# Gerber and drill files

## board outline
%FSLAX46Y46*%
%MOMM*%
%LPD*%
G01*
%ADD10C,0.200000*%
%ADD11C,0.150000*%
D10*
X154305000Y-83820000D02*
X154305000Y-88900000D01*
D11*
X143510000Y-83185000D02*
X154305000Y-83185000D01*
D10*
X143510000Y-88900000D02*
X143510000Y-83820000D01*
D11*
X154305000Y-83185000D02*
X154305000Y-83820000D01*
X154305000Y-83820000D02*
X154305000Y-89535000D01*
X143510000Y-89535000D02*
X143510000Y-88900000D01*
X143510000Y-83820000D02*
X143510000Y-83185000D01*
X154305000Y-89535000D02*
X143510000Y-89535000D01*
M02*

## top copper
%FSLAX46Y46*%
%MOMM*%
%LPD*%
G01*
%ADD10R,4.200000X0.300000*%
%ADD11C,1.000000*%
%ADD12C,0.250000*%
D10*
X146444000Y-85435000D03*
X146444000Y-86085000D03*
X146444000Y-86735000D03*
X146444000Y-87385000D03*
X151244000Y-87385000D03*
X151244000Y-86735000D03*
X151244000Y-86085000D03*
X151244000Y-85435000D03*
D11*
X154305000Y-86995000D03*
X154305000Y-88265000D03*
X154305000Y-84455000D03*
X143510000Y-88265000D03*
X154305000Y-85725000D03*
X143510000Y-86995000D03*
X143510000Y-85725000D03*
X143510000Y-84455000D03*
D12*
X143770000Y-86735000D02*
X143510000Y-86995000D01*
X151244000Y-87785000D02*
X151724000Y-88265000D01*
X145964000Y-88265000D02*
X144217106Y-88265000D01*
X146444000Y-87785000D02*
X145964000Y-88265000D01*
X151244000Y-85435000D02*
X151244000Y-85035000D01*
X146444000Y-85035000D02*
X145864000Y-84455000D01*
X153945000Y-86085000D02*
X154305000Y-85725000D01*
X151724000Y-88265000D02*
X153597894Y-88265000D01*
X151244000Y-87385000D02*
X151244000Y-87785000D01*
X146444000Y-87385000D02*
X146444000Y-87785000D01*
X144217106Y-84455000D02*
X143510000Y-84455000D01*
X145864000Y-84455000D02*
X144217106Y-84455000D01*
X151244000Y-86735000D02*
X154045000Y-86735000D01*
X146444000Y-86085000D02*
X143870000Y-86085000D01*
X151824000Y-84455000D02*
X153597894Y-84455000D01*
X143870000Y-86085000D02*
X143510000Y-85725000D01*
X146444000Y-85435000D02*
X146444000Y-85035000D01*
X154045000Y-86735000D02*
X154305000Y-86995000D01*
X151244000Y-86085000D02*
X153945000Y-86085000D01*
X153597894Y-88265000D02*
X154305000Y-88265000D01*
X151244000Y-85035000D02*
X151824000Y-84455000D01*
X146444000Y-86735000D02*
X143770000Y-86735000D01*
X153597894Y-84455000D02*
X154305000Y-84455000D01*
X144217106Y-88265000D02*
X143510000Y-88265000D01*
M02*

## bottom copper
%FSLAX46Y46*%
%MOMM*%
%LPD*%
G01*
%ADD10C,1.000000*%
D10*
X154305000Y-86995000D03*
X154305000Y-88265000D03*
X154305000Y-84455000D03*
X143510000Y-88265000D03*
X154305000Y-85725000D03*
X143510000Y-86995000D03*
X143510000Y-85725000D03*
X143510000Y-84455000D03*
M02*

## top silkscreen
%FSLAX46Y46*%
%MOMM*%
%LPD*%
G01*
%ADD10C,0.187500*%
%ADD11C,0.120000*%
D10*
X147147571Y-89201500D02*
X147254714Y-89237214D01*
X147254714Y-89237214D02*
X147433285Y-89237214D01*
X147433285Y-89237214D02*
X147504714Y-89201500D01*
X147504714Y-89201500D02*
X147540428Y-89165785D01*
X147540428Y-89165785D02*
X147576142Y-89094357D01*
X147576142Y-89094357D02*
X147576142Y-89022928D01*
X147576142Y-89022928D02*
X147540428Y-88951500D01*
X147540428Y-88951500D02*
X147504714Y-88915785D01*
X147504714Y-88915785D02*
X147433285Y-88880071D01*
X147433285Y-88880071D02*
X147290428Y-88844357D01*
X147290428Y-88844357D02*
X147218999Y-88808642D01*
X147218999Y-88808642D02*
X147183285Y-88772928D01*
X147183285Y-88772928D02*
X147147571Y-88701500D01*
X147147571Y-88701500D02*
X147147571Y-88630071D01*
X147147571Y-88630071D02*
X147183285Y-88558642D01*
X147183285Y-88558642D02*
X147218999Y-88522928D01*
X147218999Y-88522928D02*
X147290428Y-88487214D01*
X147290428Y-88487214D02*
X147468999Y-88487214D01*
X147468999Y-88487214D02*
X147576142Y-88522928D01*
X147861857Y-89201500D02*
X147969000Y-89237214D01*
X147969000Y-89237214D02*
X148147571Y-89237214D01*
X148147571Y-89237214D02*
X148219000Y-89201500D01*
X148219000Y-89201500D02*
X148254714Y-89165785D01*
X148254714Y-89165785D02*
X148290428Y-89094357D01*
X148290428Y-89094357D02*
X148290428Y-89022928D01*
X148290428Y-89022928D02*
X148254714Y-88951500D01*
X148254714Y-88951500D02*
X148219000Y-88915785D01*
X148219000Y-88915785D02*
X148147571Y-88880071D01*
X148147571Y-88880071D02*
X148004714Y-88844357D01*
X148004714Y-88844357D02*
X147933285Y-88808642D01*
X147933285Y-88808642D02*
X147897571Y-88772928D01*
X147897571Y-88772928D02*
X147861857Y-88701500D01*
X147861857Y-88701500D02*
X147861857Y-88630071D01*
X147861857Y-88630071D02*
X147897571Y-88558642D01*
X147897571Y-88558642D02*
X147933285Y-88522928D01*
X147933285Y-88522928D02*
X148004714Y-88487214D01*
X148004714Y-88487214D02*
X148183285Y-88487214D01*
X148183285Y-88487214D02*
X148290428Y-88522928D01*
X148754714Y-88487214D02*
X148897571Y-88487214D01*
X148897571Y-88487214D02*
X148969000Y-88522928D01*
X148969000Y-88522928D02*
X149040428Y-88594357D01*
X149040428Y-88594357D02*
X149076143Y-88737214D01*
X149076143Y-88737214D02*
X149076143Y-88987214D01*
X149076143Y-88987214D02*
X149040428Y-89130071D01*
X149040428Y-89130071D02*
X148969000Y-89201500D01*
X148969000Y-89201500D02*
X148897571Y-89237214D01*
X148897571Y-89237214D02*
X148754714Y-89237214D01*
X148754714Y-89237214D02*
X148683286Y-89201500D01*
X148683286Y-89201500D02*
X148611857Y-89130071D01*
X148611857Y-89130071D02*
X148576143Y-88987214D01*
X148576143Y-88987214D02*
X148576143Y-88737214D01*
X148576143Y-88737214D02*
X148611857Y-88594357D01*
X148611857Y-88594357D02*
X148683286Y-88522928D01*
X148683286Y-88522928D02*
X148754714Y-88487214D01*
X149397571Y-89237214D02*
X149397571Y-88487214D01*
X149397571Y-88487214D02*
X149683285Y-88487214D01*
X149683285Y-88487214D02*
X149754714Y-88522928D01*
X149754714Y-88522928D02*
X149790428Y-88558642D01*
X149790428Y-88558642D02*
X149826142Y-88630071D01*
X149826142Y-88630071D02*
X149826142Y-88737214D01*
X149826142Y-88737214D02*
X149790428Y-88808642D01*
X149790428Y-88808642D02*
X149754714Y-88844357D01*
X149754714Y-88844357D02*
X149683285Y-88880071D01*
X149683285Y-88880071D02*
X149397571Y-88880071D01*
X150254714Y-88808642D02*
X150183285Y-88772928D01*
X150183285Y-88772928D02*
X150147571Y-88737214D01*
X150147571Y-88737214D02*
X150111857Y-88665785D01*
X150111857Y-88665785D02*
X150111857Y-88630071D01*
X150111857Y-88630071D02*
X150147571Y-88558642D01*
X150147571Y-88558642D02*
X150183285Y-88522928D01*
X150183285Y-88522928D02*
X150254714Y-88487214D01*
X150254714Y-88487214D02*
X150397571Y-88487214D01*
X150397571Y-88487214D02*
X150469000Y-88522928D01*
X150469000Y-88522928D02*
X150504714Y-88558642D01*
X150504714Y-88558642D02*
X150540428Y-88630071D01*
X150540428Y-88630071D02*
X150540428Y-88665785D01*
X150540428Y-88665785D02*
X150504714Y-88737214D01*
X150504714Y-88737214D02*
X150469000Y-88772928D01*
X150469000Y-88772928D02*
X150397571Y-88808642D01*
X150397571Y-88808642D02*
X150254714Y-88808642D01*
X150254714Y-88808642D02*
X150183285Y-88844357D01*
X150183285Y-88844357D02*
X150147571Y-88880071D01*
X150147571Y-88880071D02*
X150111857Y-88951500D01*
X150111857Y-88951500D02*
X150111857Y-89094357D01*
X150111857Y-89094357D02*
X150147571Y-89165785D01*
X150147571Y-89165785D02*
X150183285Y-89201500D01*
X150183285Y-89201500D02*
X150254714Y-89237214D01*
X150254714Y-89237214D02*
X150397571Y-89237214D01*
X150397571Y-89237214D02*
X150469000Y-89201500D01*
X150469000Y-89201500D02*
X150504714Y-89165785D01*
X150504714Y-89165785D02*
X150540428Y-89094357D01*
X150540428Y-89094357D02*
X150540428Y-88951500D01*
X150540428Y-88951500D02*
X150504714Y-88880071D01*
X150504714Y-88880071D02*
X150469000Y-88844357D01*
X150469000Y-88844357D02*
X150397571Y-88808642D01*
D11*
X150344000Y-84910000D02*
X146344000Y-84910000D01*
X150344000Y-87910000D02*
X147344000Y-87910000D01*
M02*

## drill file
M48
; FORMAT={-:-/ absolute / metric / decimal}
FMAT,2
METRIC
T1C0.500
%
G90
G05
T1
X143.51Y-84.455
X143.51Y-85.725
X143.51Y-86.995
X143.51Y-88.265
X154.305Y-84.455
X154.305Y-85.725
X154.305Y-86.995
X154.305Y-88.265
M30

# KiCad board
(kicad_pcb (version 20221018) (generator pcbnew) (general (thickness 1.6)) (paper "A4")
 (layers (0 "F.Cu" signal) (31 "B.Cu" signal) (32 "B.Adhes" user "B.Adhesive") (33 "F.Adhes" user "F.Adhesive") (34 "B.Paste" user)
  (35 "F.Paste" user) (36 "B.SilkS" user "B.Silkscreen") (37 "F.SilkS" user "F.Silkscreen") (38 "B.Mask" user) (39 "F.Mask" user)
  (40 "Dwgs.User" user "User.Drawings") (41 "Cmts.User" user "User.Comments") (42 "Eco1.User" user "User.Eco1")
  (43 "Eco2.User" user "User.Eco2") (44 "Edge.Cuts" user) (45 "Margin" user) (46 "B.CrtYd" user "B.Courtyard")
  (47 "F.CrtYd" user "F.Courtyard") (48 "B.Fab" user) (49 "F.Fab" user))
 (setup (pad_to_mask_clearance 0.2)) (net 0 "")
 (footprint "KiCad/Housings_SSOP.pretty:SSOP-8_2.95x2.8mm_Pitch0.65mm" (layer "F.Cu") (at 148.844 86.41)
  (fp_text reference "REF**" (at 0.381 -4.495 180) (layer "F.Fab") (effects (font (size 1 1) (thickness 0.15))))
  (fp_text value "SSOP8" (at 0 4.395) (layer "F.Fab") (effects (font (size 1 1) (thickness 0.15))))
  (fp_line (start 1.5 -1.5) (end -2.5 -1.5) (stroke (width 0.12) (type solid)) (layer "F.SilkS"))
  (fp_line (start 1.5 1.5) (end -1.5 1.5) (stroke (width 0.12) (type solid)) (layer "F.SilkS"))
  (pad "1" smd rect (at -2.4 -0.975 270) (size 0.3 4.2) (layers "F.Cu" "F.Paste" "F.Mask"))
  (pad "2" smd rect (at -2.4 -0.325 270) (size 0.3 4.2) (layers "F.Cu" "F.Paste" "F.Mask"))
  (pad "3" smd rect (at -2.4 0.325 270) (size 0.3 4.2) (layers "F.Cu" "F.Paste" "F.Mask"))
  (pad "4" smd rect (at -2.4 0.975 270) (size 0.3 4.2) (layers "F.Cu" "F.Paste" "F.Mask"))
  (pad "5" smd rect (at 2.4 0.975 270) (size 0.3 4.2) (layers "F.Cu" "F.Paste" "F.Mask"))
  (pad "6" smd rect (at 2.4 0.325 270) (size 0.3 4.2) (layers "F.Cu" "F.Paste" "F.Mask"))
  (pad "7" smd rect (at 2.4 -0.325 270) (size 0.3 4.2) (layers "F.Cu" "F.Paste" "F.Mask"))
  (pad "8" smd rect (at 2.4 -0.975 270) (size 0.3 4.2) (layers "F.Cu" "F.Paste" "F.Mask")))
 (gr_line (start 154.305 83.82) (end 154.305 88.9) (stroke (width 0.2) (type solid)) (layer "Edge.Cuts"))
 (gr_line (start 143.51 83.185) (end 154.305 83.185) (stroke (width 0.15) (type solid)) (layer "Edge.Cuts"))
 (gr_line (start 143.51 88.9) (end 143.51 83.82) (stroke (width 0.2) (type solid)) (layer "Edge.Cuts"))
 (gr_line (start 154.305 83.185) (end 154.305 83.82) (stroke (width 0.15) (type solid)) (layer "Edge.Cuts"))
 (gr_line (start 154.305 83.82) (end 154.305 89.535) (stroke (width 0.15) (type solid)) (layer "Edge.Cuts"))
 (gr_line (start 143.51 89.535) (end 143.51 88.9) (stroke (width 0.15) (type solid)) (layer "Edge.Cuts"))
 (gr_line (start 143.51 83.82) (end 143.51 83.185) (stroke (width 0.15) (type solid)) (layer "Edge.Cuts"))
 (gr_line (start 154.305 89.535) (end 143.51 89.535) (stroke (width 0.15) (type solid)) (layer "Edge.Cuts"))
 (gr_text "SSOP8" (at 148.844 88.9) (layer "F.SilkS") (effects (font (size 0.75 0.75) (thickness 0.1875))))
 (segment (start 143.77 86.735) (end 143.51 86.995) (width 0.25) (layer "F.Cu") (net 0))
 (segment (start 151.244 87.785) (end 151.724 88.265) (width 0.25) (layer "F.Cu") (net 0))
 (segment (start 145.964 88.265) (end 144.217106 88.265) (width 0.25) (layer "F.Cu") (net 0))
 (segment (start 146.444 87.785) (end 145.964 88.265) (width 0.25) (layer "F.Cu") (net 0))
 (segment (start 151.244 85.435) (end 151.244 85.035) (width 0.25) (layer "F.Cu") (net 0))
 (segment (start 146.444 85.035) (end 145.864 84.455) (width 0.25) (layer "F.Cu") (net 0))
 (segment (start 153.945 86.085) (end 154.305 85.725) (width 0.25) (layer "F.Cu") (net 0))
 (segment (start 151.724 88.265) (end 153.597894 88.265) (width 0.25) (layer "F.Cu") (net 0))
 (segment (start 151.244 87.385) (end 151.244 87.785) (width 0.25) (layer "F.Cu") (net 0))
 (segment (start 146.444 87.385) (end 146.444 87.785) (width 0.25) (layer "F.Cu") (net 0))
 (segment (start 144.217106 84.455) (end 143.51 84.455) (width 0.25) (layer "F.Cu") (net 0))
 (segment (start 145.864 84.455) (end 144.217106 84.455) (width 0.25) (layer "F.Cu") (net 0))
 (segment (start 151.244 86.735) (end 154.045 86.735) (width 0.25) (layer "F.Cu") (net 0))
 (segment (start 146.444 86.085) (end 143.87 86.085) (width 0.25) (layer "F.Cu") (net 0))
 (segment (start 151.824 84.455) (end 153.597894 84.455) (width 0.25) (layer "F.Cu") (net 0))
 (segment (start 143.87 86.085) (end 143.51 85.725) (width 0.25) (layer "F.Cu") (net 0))
 (segment (start 146.444 85.435) (end 146.444 85.035) (width 0.25) (layer "F.Cu") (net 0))
 (segment (start 154.045 86.735) (end 154.305 86.995) (width 0.25) (layer "F.Cu") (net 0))
 (segment (start 151.244 86.085) (end 153.945 86.085) (width 0.25) (layer "F.Cu") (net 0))
 (segment (start 153.597894 88.265) (end 154.305 88.265) (width 0.25) (layer "F.Cu") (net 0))
 (segment (start 151.244 85.035) (end 151.824 84.455) (width 0.25) (layer "F.Cu") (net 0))
 (segment (start 146.444 86.735) (end 143.77 86.735) (width 0.25) (layer "F.Cu") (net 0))
 (segment (start 153.597894 84.455) (end 154.305 84.455) (width 0.25) (layer "F.Cu") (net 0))
 (segment (start 144.217106 88.265) (end 143.51 88.265) (width 0.25) (layer "F.Cu") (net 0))
 (via (at 154.305 86.995) (size 1) (drill 0.5) (layers "F.Cu" "B.Cu") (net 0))
 (via (at 154.305 88.265) (size 1) (drill 0.5) (layers "F.Cu" "B.Cu") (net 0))
 (via (at 154.305 84.455) (size 1) (drill 0.5) (layers "F.Cu" "B.Cu") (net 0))
 (via (at 143.51 88.265) (size 1) (drill 0.5) (layers "F.Cu" "B.Cu") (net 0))
 (via (at 154.305 85.725) (size 1) (drill 0.5) (layers "F.Cu" "B.Cu") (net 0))
 (via (at 143.51 86.995) (size 1) (drill 0.5) (layers "F.Cu" "B.Cu") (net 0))
 (via (at 143.51 85.725) (size 1) (drill 0.5) (layers "F.Cu" "B.Cu") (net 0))
 (via (at 143.51 84.455) (size 1) (drill 0.5) (layers "F.Cu" "B.Cu") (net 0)))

